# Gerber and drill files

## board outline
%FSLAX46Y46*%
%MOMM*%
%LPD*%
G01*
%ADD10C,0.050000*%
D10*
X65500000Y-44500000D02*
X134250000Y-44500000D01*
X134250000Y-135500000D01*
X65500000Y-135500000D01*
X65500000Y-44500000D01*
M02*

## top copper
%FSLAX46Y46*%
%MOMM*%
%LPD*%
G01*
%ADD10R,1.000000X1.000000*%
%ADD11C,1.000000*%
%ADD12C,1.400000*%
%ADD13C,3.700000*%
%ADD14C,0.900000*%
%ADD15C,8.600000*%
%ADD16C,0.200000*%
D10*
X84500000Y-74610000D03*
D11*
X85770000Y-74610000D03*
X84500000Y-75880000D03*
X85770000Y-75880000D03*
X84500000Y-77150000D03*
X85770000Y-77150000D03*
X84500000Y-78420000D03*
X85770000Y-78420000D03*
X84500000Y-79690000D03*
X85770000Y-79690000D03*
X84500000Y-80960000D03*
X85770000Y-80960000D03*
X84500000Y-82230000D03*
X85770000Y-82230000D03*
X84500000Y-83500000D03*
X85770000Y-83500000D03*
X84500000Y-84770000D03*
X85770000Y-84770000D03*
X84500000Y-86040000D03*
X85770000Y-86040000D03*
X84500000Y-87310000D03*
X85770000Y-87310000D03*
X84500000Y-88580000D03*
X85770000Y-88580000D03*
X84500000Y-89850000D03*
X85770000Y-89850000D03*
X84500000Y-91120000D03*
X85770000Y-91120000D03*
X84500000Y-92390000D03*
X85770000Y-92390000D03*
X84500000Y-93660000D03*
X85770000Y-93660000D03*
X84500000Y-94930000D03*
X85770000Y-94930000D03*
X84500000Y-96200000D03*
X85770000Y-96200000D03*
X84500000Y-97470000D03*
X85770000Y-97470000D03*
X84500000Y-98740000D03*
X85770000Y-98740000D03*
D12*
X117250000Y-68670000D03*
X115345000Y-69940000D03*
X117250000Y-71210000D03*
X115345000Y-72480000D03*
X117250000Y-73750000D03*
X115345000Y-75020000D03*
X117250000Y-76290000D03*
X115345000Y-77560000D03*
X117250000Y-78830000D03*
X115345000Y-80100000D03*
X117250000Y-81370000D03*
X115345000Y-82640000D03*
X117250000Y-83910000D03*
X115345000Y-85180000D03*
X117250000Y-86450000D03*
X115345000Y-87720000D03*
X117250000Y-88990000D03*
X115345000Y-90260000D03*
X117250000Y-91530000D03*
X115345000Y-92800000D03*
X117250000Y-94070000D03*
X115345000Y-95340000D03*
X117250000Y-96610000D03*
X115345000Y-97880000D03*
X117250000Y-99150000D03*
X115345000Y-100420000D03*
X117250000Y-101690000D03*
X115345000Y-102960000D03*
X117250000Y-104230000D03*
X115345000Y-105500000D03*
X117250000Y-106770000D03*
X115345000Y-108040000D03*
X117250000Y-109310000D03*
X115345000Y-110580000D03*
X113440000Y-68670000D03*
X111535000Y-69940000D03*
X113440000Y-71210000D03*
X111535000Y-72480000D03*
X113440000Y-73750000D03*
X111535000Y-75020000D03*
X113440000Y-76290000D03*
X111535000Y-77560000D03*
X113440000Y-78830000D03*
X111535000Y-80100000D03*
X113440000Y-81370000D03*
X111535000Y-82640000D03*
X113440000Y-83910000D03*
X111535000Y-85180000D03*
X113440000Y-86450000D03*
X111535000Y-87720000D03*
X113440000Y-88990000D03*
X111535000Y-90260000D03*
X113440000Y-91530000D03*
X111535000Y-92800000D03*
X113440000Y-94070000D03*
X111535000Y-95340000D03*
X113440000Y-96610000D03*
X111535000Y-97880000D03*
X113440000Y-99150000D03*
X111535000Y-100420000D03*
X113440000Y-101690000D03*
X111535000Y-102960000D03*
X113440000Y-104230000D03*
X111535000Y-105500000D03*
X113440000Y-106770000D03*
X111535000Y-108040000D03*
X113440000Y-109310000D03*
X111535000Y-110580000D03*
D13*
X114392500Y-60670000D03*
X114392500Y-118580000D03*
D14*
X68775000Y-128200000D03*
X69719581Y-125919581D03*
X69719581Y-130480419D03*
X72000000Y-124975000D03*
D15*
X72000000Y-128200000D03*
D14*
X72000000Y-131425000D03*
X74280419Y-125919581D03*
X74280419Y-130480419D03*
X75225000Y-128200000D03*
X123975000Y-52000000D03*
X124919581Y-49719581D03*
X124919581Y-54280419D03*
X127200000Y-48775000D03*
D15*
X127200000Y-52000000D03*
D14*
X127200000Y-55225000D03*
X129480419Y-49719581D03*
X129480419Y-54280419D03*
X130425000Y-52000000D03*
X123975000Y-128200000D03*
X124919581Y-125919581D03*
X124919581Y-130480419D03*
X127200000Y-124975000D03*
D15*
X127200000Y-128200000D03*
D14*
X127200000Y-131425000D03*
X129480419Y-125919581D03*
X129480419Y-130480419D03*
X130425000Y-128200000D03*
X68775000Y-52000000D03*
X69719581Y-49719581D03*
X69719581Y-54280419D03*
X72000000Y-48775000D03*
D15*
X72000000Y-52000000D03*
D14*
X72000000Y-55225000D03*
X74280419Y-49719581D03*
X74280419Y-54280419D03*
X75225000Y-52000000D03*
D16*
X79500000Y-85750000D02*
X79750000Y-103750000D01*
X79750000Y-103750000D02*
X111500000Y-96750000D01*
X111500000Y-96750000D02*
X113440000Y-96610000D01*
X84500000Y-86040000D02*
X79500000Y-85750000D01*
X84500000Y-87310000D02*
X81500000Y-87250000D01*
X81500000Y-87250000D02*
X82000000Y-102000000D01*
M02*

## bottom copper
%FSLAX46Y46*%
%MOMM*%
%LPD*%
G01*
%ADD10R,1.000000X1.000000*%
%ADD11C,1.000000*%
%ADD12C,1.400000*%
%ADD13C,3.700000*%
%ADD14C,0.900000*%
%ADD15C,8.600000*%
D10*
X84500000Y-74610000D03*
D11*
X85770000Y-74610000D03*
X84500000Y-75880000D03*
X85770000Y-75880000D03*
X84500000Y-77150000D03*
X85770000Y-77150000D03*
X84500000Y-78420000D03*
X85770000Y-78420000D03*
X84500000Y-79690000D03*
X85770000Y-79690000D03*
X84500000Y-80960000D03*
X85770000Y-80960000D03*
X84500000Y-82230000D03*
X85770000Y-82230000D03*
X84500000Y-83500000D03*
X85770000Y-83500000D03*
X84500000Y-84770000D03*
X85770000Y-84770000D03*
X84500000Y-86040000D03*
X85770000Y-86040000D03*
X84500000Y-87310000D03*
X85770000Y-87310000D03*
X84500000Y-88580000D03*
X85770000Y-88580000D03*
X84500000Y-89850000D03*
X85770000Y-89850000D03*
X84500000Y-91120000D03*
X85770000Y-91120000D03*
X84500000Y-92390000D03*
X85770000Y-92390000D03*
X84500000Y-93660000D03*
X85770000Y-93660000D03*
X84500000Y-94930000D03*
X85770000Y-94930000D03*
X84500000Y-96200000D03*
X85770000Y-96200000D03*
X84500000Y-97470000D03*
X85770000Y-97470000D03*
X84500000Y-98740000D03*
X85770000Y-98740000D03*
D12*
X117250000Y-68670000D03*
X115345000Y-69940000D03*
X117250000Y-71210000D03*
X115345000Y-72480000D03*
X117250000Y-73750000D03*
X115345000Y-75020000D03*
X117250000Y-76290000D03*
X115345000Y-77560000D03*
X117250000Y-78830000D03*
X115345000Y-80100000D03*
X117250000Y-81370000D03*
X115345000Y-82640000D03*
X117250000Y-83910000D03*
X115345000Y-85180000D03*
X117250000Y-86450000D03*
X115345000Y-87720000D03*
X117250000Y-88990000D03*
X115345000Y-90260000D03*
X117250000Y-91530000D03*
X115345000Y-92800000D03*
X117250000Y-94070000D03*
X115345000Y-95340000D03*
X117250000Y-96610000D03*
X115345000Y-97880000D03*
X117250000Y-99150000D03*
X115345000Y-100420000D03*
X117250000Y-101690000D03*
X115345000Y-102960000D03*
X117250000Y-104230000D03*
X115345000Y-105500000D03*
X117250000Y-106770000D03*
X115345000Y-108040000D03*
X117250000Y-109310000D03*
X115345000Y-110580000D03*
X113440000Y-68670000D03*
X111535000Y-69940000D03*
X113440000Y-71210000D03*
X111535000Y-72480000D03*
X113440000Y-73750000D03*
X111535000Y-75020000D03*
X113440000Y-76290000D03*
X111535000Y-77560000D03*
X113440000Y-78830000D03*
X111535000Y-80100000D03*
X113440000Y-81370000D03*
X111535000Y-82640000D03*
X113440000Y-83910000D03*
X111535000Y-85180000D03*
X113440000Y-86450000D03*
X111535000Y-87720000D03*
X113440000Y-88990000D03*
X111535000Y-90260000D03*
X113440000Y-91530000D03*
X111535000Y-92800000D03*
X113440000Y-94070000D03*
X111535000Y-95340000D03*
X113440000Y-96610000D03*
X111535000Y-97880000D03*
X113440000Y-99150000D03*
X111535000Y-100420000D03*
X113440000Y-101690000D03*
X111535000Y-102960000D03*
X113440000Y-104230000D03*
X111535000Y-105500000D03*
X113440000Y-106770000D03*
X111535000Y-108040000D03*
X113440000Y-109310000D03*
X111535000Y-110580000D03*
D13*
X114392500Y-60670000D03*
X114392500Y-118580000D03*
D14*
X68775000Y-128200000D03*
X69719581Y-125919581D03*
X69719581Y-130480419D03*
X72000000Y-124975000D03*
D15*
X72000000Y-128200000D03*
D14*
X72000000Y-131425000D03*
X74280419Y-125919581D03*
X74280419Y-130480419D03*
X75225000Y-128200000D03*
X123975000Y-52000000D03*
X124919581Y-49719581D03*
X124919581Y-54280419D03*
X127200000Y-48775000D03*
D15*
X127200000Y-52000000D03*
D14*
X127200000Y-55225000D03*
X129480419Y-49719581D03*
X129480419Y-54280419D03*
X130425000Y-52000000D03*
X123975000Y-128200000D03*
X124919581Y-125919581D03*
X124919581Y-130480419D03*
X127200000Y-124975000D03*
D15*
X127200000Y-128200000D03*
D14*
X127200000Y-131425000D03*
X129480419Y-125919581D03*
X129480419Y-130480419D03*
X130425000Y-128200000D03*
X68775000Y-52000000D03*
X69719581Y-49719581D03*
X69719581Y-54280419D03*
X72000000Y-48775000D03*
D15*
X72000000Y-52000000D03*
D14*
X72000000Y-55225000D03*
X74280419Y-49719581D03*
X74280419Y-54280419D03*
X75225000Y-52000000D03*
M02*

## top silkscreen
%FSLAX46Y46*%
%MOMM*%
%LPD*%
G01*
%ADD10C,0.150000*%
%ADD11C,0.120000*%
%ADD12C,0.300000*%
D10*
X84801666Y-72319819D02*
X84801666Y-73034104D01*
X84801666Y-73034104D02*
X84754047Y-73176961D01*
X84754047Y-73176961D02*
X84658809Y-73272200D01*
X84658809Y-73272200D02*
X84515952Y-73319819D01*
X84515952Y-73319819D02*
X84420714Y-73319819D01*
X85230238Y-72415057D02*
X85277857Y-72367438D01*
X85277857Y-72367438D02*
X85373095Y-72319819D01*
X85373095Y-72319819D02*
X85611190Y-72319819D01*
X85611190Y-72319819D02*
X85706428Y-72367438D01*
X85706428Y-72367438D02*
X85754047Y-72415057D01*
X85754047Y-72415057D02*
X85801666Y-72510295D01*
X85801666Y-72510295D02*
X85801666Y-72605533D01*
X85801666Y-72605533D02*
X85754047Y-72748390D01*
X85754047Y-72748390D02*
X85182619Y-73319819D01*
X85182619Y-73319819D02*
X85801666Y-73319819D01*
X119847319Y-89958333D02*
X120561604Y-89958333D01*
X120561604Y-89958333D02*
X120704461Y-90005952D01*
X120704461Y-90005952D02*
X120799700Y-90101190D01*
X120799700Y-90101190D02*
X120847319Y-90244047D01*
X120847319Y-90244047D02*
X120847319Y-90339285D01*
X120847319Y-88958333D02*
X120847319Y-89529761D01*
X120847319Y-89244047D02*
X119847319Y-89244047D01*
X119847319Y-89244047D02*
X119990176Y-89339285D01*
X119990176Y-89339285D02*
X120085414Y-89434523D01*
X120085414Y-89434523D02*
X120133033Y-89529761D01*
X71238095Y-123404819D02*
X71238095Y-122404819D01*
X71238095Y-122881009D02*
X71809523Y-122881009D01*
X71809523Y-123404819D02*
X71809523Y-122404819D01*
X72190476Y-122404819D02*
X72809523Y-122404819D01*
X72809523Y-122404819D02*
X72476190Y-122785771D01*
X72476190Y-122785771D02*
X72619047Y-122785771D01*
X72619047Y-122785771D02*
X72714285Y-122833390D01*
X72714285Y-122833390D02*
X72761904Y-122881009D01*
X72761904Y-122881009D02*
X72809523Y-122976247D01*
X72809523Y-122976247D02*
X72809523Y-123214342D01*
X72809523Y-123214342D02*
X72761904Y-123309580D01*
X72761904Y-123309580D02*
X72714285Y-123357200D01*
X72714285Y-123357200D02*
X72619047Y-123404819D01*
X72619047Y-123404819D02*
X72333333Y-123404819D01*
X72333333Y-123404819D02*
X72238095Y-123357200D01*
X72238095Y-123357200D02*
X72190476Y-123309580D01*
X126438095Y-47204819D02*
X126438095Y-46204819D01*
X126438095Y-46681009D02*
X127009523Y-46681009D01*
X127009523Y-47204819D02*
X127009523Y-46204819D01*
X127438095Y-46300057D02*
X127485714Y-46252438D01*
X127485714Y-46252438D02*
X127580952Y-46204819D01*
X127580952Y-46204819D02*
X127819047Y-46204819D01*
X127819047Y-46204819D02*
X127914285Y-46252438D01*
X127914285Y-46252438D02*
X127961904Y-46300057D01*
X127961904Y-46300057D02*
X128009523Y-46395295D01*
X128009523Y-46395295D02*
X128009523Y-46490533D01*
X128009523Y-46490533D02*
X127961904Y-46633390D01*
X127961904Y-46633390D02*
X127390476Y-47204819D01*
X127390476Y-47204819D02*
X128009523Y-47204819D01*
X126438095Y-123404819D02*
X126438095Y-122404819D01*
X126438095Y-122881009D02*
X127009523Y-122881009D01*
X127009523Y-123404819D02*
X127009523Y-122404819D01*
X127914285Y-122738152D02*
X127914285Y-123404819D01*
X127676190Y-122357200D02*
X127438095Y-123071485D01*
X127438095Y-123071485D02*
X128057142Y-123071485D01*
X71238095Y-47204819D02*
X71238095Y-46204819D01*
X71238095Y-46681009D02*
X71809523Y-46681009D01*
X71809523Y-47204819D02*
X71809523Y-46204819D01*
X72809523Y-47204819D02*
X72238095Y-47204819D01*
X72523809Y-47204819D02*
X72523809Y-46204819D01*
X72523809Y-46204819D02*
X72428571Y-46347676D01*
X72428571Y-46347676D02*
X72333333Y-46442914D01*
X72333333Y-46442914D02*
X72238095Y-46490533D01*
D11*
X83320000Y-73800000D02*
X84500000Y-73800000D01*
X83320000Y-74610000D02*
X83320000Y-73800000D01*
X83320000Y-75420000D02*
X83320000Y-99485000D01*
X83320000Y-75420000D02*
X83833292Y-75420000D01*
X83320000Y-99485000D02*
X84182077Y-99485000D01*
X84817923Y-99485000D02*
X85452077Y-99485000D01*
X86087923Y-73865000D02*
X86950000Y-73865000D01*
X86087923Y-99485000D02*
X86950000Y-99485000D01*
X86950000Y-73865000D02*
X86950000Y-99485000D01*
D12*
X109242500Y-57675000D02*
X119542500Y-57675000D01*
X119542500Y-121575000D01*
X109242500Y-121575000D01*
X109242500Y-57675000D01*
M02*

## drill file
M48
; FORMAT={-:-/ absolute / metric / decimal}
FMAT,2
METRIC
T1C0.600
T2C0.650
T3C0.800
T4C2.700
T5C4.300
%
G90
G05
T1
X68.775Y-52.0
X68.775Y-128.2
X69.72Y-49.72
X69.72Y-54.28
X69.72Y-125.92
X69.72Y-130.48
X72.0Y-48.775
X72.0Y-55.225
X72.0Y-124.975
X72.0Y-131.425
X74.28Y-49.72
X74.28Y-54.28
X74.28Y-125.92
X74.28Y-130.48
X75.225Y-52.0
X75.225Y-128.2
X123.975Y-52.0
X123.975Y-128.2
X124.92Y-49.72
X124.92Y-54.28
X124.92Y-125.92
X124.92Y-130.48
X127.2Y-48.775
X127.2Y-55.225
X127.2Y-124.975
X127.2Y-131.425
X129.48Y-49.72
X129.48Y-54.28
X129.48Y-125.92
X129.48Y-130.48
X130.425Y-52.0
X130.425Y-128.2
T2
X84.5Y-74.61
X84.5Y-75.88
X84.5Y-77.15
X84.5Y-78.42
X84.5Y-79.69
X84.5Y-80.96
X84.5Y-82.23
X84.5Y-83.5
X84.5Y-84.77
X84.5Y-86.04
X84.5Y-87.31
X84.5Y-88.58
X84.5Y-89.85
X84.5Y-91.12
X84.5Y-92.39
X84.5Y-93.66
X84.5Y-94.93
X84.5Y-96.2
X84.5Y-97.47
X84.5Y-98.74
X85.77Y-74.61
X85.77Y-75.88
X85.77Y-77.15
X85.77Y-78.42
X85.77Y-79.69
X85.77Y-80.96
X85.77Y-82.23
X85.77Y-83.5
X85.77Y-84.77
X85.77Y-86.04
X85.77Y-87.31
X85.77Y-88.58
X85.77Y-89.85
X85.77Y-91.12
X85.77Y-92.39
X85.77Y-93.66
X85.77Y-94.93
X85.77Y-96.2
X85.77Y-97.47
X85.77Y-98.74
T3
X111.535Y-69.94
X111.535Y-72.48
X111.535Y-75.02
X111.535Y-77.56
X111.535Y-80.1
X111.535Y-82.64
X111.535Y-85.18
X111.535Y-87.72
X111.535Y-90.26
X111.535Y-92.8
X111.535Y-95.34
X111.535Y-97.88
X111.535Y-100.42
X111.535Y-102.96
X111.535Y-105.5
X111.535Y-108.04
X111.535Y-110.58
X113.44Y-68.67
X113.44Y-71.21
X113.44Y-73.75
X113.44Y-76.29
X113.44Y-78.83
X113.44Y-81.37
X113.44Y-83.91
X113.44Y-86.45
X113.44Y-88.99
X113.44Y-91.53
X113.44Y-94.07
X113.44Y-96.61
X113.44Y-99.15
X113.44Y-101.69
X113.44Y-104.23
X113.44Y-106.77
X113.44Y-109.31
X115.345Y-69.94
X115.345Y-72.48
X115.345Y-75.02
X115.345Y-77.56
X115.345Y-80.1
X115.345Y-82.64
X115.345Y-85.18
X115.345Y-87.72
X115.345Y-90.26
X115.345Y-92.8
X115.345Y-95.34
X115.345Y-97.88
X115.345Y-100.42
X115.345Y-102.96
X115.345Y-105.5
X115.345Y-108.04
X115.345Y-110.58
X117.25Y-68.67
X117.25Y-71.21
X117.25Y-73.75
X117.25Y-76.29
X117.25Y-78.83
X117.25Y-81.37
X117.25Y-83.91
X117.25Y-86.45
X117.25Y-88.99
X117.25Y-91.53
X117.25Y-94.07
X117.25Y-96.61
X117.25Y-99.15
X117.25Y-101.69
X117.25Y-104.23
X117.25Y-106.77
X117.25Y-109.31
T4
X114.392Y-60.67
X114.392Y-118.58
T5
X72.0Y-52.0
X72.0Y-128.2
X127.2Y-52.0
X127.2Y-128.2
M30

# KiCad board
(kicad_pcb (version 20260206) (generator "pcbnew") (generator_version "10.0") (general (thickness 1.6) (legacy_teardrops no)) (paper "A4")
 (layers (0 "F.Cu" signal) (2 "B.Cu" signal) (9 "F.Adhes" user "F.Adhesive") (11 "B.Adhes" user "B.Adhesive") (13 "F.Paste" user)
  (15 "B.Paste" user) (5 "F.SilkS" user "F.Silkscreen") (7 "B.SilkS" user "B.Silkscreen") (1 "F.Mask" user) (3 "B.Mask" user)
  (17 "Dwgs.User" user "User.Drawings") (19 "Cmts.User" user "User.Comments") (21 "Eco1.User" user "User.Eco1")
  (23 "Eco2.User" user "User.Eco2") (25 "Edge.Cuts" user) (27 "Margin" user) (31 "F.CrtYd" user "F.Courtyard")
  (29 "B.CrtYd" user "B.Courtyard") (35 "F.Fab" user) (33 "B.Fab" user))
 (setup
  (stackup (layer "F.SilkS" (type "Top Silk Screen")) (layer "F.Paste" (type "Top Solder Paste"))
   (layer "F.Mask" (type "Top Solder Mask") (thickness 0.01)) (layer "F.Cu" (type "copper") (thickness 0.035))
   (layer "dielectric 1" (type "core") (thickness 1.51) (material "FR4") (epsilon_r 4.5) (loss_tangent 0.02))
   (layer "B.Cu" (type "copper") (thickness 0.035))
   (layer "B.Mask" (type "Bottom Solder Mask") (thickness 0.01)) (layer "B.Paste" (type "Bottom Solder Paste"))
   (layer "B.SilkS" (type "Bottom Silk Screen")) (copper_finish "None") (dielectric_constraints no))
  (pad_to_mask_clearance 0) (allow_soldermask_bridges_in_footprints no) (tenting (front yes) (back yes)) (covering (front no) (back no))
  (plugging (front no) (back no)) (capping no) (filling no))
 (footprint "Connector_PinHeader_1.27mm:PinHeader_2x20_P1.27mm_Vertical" (layer "F.Cu") (at 84.5 74.61)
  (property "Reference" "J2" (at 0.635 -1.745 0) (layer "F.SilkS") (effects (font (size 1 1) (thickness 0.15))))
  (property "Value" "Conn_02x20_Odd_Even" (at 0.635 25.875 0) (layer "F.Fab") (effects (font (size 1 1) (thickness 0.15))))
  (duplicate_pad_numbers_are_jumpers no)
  (fp_line (start -1.18 -0.81) (end 0 -0.81) (stroke (width 0.12) (type solid)) (layer "F.SilkS"))
  (fp_line (start -1.18 0) (end -1.18 -0.81) (stroke (width 0.12) (type solid)) (layer "F.SilkS"))
  (fp_line (start -1.18 0.81) (end -1.18 24.875) (stroke (width 0.12) (type solid)) (layer "F.SilkS"))
  (fp_line (start -1.18 0.81) (end -0.666708 0.81) (stroke (width 0.12) (type solid)) (layer "F.SilkS"))
  (fp_line (start -1.18 24.875) (end -0.317923 24.875) (stroke (width 0.12) (type solid)) (layer "F.SilkS"))
  (fp_line (start 0.317923 24.875) (end 0.952077 24.875) (stroke (width 0.12) (type solid)) (layer "F.SilkS"))
  (fp_line (start 1.587923 -0.745) (end 2.45 -0.745) (stroke (width 0.12) (type solid)) (layer "F.SilkS"))
  (fp_line (start 1.587923 24.875) (end 2.45 24.875) (stroke (width 0.12) (type solid)) (layer "F.SilkS"))
  (fp_line (start 2.45 -0.745) (end 2.45 24.875) (stroke (width 0.12) (type solid)) (layer "F.SilkS"))
  (pad "1" thru_hole rect (at 0 0) (size 1 1) (drill 0.65) (layers "*.Cu" "*.Mask") (remove_unused_layers no) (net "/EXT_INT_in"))
  (pad "2" thru_hole circle (at 1.27 0) (size 1 1) (drill 0.65) (layers "*.Cu" "*.Mask") (remove_unused_layers no) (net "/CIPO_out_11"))
  (pad "3" thru_hole circle (at 0 1.27) (size 1 1) (drill 0.65) (layers "*.Cu" "*.Mask") (remove_unused_layers no) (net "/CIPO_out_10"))
  (pad "4" thru_hole circle (at 1.27 1.27) (size 1 1) (drill 0.65) (layers "*.Cu" "*.Mask") (remove_unused_layers no) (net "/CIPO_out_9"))
  (pad "5" thru_hole circle (at 0 2.54) (size 1 1) (drill 0.65) (layers "*.Cu" "*.Mask") (remove_unused_layers no) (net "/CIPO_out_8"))
  (pad "6" thru_hole circle (at 1.27 2.54) (size 1 1) (drill 0.65) (layers "*.Cu" "*.Mask") (remove_unused_layers no) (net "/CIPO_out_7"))
  (pad "7" thru_hole circle (at 0 3.81) (size 1 1) (drill 0.65) (layers "*.Cu" "*.Mask") (remove_unused_layers no) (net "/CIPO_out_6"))
  (pad "8" thru_hole circle (at 1.27 3.81) (size 1 1) (drill 0.65) (layers "*.Cu" "*.Mask") (remove_unused_layers no) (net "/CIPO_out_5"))
  (pad "9" thru_hole circle (at 0 5.08) (size 1 1) (drill 0.65) (layers "*.Cu" "*.Mask") (remove_unused_layers no) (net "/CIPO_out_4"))
  (pad "10" thru_hole circle (at 1.27 5.08) (size 1 1) (drill 0.65) (layers "*.Cu" "*.Mask") (remove_unused_layers no) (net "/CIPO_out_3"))
  (pad "11" thru_hole circle (at 0 6.35) (size 1 1) (drill 0.65) (layers "*.Cu" "*.Mask") (remove_unused_layers no) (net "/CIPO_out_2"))
  (pad "12" thru_hole circle (at 1.27 6.35) (size 1 1) (drill 0.65) (layers "*.Cu" "*.Mask") (remove_unused_layers no) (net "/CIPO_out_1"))
  (pad "13" thru_hole circle (at 0 7.62) (size 1 1) (drill 0.65) (layers "*.Cu" "*.Mask") (remove_unused_layers no) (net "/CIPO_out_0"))
  (pad "14" thru_hole circle (at 1.27 7.62) (size 1 1) (drill 0.65) (layers "*.Cu" "*.Mask") (remove_unused_layers no) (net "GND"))
  (pad "15" thru_hole circle (at 0 8.89) (size 1 1) (drill 0.65) (layers "*.Cu" "*.Mask") (remove_unused_layers no) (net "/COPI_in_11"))
  (pad "16" thru_hole circle (at 1.27 8.89) (size 1 1) (drill 0.65) (layers "*.Cu" "*.Mask") (remove_unused_layers no) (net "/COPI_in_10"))
  (pad "17" thru_hole circle (at 0 10.16) (size 1 1) (drill 0.65) (layers "*.Cu" "*.Mask") (remove_unused_layers no) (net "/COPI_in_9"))
  (pad "18" thru_hole circle (at 1.27 10.16) (size 1 1) (drill 0.65) (layers "*.Cu" "*.Mask") (remove_unused_layers no) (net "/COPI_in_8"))
  (pad "19" thru_hole circle (at 0 11.43) (size 1 1) (drill 0.65) (layers "*.Cu" "*.Mask") (remove_unused_layers no) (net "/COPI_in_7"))
  (pad "20" thru_hole circle (at 1.27 11.43) (size 1 1) (drill 0.65) (layers "*.Cu" "*.Mask") (remove_unused_layers no) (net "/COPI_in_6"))
  (pad "21" thru_hole circle (at 0 12.7) (size 1 1) (drill 0.65) (layers "*.Cu" "*.Mask") (remove_unused_layers no) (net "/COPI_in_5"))
  (pad "22" thru_hole circle (at 1.27 12.7) (size 1 1) (drill 0.65) (layers "*.Cu" "*.Mask") (remove_unused_layers no) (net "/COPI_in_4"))
  (pad "23" thru_hole circle (at 0 13.97) (size 1 1) (drill 0.65) (layers "*.Cu" "*.Mask") (remove_unused_layers no) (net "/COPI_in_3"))
  (pad "24" thru_hole circle (at 1.27 13.97) (size 1 1) (drill 0.65) (layers "*.Cu" "*.Mask") (remove_unused_layers no) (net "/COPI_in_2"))
  (pad "25" thru_hole circle (at 0 15.24) (size 1 1) (drill 0.65) (layers "*.Cu" "*.Mask") (remove_unused_layers no) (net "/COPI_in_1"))
  (pad "26" thru_hole circle (at 1.27 15.24) (size 1 1) (drill 0.65) (layers "*.Cu" "*.Mask") (remove_unused_layers no) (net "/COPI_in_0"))
  (pad "27" thru_hole circle (at 0 16.51) (size 1 1) (drill 0.65) (layers "*.Cu" "*.Mask") (remove_unused_layers no) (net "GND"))
  (pad "28" thru_hole circle (at 1.27 16.51) (size 1 1) (drill 0.65) (layers "*.Cu" "*.Mask") (remove_unused_layers no) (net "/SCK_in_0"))
  (pad "29" thru_hole circle (at 0 17.78) (size 1 1) (drill 0.65) (layers "*.Cu" "*.Mask") (remove_unused_layers no) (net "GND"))
  (pad "30" thru_hole circle (at 1.27 17.78) (size 1 1) (drill 0.65) (layers "*.Cu" "*.Mask") (remove_unused_layers no) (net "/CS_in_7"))
  (pad "31" thru_hole circle (at 0 19.05) (size 1 1) (drill 0.65) (layers "*.Cu" "*.Mask") (remove_unused_layers no) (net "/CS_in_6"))
  (pad "32" thru_hole circle (at 1.27 19.05) (size 1 1) (drill 0.65) (layers "*.Cu" "*.Mask") (remove_unused_layers no) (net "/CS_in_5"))
  (pad "33" thru_hole circle (at 0 20.32) (size 1 1) (drill 0.65) (layers "*.Cu" "*.Mask") (remove_unused_layers no) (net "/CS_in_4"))
  (pad "34" thru_hole circle (at 1.27 20.32) (size 1 1) (drill 0.65) (layers "*.Cu" "*.Mask") (remove_unused_layers no) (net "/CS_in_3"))
  (pad "35" thru_hole circle (at 0 21.59) (size 1 1) (drill 0.65) (layers "*.Cu" "*.Mask") (remove_unused_layers no) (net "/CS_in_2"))
  (pad "36" thru_hole circle (at 1.27 21.59) (size 1 1) (drill 0.65) (layers "*.Cu" "*.Mask") (remove_unused_layers no) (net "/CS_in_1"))
  (pad "37" thru_hole circle (at 0 22.86) (size 1 1) (drill 0.65) (layers "*.Cu" "*.Mask") (remove_unused_layers no) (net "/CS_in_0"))
  (pad "38" thru_hole circle (at 1.27 22.86) (size 1 1) (drill 0.65) (layers "*.Cu" "*.Mask") (remove_unused_layers no) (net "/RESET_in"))
  (pad "39" thru_hole circle (at 0 24.13) (size 1 1) (drill 0.65) (layers "*.Cu" "*.Mask") (remove_unused_layers no) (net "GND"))
  (pad "40" thru_hole circle (at 1.27 24.13) (size 1 1) (drill 0.65) (layers "*.Cu" "*.Mask") (remove_unused_layers no) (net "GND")))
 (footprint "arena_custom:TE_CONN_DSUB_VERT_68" (layer "F.Cu") (at 114.3925 89.625 -90)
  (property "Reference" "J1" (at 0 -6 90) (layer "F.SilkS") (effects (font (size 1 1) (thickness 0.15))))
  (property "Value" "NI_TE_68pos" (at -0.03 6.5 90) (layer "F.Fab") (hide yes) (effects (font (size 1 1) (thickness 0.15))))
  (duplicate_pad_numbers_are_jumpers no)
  (fp_rect (start -31.95 -5.15) (end 31.95 5.15) (stroke (width 0.3) (type default)) (fill no) (layer "F.SilkS"))
  (pad "1" thru_hole circle (at -20.955 -2.8575 270) (size 1.4 1.4) (drill 0.8) (layers "*.Cu" "*.Mask") (remove_unused_layers no)
   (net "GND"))
  (pad "2" thru_hole circle (at -19.685 -0.9525 270) (size 1.4 1.4) (drill 0.8) (layers "*.Cu" "*.Mask") (remove_unused_layers no)
   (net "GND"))
  (pad "3" thru_hole circle (at -18.415 -2.8575 270) (size 1.4 1.4) (drill 0.8) (layers "*.Cu" "*.Mask") (remove_unused_layers no)
   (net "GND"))
  (pad "4" thru_hole circle (at -17.145 -0.9525 270) (size 1.4 1.4) (drill 0.8) (layers "*.Cu" "*.Mask") (remove_unused_layers no)
   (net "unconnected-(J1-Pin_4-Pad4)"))
  (pad "5" thru_hole circle (at -15.875 -2.8575 270) (size 1.4 1.4) (drill 0.8) (layers "*.Cu" "*.Mask") (remove_unused_layers no)
   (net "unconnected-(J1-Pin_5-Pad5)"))
  (pad "6" thru_hole circle (at -14.605 -0.9525 270) (size 1.4 1.4) (drill 0.8) (layers "*.Cu" "*.Mask") (remove_unused_layers no)
   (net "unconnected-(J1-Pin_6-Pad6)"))
  (pad "7" thru_hole circle (at -13.335 -2.8575 270) (size 1.4 1.4) (drill 0.8) (layers "*.Cu" "*.Mask") (remove_unused_layers no)
   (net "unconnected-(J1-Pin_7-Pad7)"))
  (pad "8" thru_hole circle (at -12.065 -0.9525 270) (size 1.4 1.4) (drill 0.8) (layers "*.Cu" "*.Mask") (remove_unused_layers no)
   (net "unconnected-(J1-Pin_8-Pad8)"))
  (pad "9" thru_hole circle (at -10.795 -2.8575 270) (size 1.4 1.4) (drill 0.8) (layers "*.Cu" "*.Mask") (remove_unused_layers no)
   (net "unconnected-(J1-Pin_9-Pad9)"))
  (pad "10" thru_hole circle (at -9.525 -0.9525 270) (size 1.4 1.4) (drill 0.8) (layers "*.Cu" "*.Mask") (remove_unused_layers no)
   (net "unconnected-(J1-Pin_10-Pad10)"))
  (pad "11" thru_hole circle (at -8.255 -2.8575 270) (size 1.4 1.4) (drill 0.8) (layers "*.Cu" "*.Mask") (remove_unused_layers no)
   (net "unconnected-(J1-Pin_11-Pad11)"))
  (pad "12" thru_hole circle (at -6.985 -0.9525 270) (size 1.4 1.4) (drill 0.8) (layers "*.Cu" "*.Mask") (remove_unused_layers no)
   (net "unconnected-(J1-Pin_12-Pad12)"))
  (pad "13" thru_hole circle (at -5.715 -2.8575 270) (size 1.4 1.4) (drill 0.8) (layers "*.Cu" "*.Mask") (remove_unused_layers no)
   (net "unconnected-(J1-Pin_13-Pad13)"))
  (pad "14" thru_hole circle (at -4.445 -0.9525 270) (size 1.4 1.4) (drill 0.8) (layers "*.Cu" "*.Mask") (remove_unused_layers no)
   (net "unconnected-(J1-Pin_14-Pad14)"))
  (pad "15" thru_hole circle (at -3.175 -2.8575 270) (size 1.4 1.4) (drill 0.8) (layers "*.Cu" "*.Mask") (remove_unused_layers no)
   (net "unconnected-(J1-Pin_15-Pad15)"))
  (pad "16" thru_hole circle (at -1.905 -0.9525 270) (size 1.4 1.4) (drill 0.8) (layers "*.Cu" "*.Mask") (remove_unused_layers no)
   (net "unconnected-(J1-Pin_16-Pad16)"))
  (pad "17" thru_hole circle (at -0.635 -2.8575 270) (size 1.4 1.4) (drill 0.8) (layers "*.Cu" "*.Mask") (remove_unused_layers no)
   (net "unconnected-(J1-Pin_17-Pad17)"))
  (pad "18" thru_hole circle (at 0.635 -0.9525 270) (size 1.4 1.4) (drill 0.8) (layers "*.Cu" "*.Mask") (remove_unused_layers no)
   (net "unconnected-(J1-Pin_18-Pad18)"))
  (pad "19" thru_hole circle (at 1.905 -2.8575 270) (size 1.4 1.4) (drill 0.8) (layers "*.Cu" "*.Mask") (remove_unused_layers no)
   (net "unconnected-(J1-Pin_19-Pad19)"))
  (pad "20" thru_hole circle (at 3.175 -0.9525 270) (size 1.4 1.4) (drill 0.8) (layers "*.Cu" "*.Mask") (remove_unused_layers no)
   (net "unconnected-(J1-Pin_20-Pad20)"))
  (pad "21" thru_hole circle (at 4.445 -2.8575 270) (size 1.4 1.4) (drill 0.8) (layers "*.Cu" "*.Mask") (remove_unused_layers no)
   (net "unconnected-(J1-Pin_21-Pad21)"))
  (pad "22" thru_hole circle (at 5.715 -0.9525 270) (size 1.4 1.4) (drill 0.8) (layers "*.Cu" "*.Mask") (remove_unused_layers no)
   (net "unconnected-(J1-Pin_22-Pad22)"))
  (pad "23" thru_hole circle (at 6.985 -2.8575 270) (size 1.4 1.4) (drill 0.8) (layers "*.Cu" "*.Mask") (remove_unused_layers no)
   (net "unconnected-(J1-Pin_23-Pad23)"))
  (pad "24" thru_hole circle (at 8.255 -0.9525 270) (size 1.4 1.4) (drill 0.8) (layers "*.Cu" "*.Mask") (remove_unused_layers no)
   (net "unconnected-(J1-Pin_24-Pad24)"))
  (pad "25" thru_hole circle (at 9.525 -2.8575 270) (size 1.4 1.4) (drill 0.8) (layers "*.Cu" "*.Mask") (remove_unused_layers no)
   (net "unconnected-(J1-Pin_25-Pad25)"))
  (pad "26" thru_hole circle (at 10.795 -0.9525 270) (size 1.4 1.4) (drill 0.8) (layers "*.Cu" "*.Mask") (remove_unused_layers no)
   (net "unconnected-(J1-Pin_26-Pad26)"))
  (pad "27" thru_hole circle (at 12.065 -2.8575 270) (size 1.4 1.4) (drill 0.8) (layers "*.Cu" "*.Mask") (remove_unused_layers no)
   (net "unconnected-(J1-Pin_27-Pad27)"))
  (pad "28" thru_hole circle (at 13.335 -0.9525 270) (size 1.4 1.4) (drill 0.8) (layers "*.Cu" "*.Mask") (remove_unused_layers no)
   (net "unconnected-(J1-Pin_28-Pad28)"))
  (pad "29" thru_hole circle (at 14.605 -2.8575 270) (size 1.4 1.4) (drill 0.8) (layers "*.Cu" "*.Mask") (remove_unused_layers no)
   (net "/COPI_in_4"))
  (pad "30" thru_hole circle (at 15.875 -0.9525 270) (size 1.4 1.4) (drill 0.8) (layers "*.Cu" "*.Mask") (remove_unused_layers no)
   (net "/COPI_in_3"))
  (pad "31" thru_hole circle (at 17.145 -2.8575 270) (size 1.4 1.4) (drill 0.8) (layers "*.Cu" "*.Mask") (remove_unused_layers no)
   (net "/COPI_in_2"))
  (pad "32" thru_hole circle (at 18.415 -0.9525 270) (size 1.4 1.4) (drill 0.8) (layers "*.Cu" "*.Mask") (remove_unused_layers no)
   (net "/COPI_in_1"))
  (pad "33" thru_hole circle (at 19.685 -2.8575 270) (size 1.4 1.4) (drill 0.8) (layers "*.Cu" "*.Mask") (remove_unused_layers no)
   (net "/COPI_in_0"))
  (pad "34" thru_hole circle (at 20.955 -0.9525 270) (size 1.4 1.4) (drill 0.8) (layers "*.Cu" "*.Mask") (remove_unused_layers no)
   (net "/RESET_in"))
  (pad "35" thru_hole circle (at -20.955 0.9525 270) (size 1.4 1.4) (drill 0.8) (layers "*.Cu" "*.Mask") (remove_unused_layers no)
   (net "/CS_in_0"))
  (pad "36" thru_hole circle (at -19.685 2.8575 270) (size 1.4 1.4) (drill 0.8) (layers "*.Cu" "*.Mask") (remove_unused_layers no)
   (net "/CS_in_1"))
  (pad "37" thru_hole circle (at -18.415 0.9525 270) (size 1.4 1.4) (drill 0.8) (layers "*.Cu" "*.Mask") (remove_unused_layers no)
   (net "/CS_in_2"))
  (pad "38" thru_hole circle (at -17.145 2.8575 270) (size 1.4 1.4) (drill 0.8) (layers "*.Cu" "*.Mask") (remove_unused_layers no)
   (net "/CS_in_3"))
  (pad "39" thru_hole circle (at -15.875 0.9525 270) (size 1.4 1.4) (drill 0.8) (layers "*.Cu" "*.Mask") (remove_unused_layers no)
   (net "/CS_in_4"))
  (pad "40" thru_hole circle (at -14.605 2.8575 270) (size 1.4 1.4) (drill 0.8) (layers "*.Cu" "*.Mask") (remove_unused_layers no)
   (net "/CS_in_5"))
  (pad "41" thru_hole circle (at -13.335 0.9525 270) (size 1.4 1.4) (drill 0.8) (layers "*.Cu" "*.Mask") (remove_unused_layers no)
   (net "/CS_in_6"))
  (pad "42" thru_hole circle (at -12.065 2.8575 270) (size 1.4 1.4) (drill 0.8) (layers "*.Cu" "*.Mask") (remove_unused_layers no)
   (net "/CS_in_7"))
  (pad "43" thru_hole circle (at -10.795 0.9525 270) (size 1.4 1.4) (drill 0.8) (layers "*.Cu" "*.Mask") (remove_unused_layers no)
   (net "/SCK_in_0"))
  (pad "44" thru_hole circle (at -9.525 2.8575 270) (size 1.4 1.4) (drill 0.8) (layers "*.Cu" "*.Mask") (remove_unused_layers no)
   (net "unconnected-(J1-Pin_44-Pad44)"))
  (pad "45" thru_hole circle (at -8.255 0.9525 270) (size 1.4 1.4) (drill 0.8) (layers "*.Cu" "*.Mask") (remove_unused_layers no)
   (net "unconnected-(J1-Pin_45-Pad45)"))
  (pad "46" thru_hole circle (at -6.985 2.8575 270) (size 1.4 1.4) (drill 0.8) (layers "*.Cu" "*.Mask") (remove_unused_layers no)
   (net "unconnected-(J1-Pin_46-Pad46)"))
  (pad "47" thru_hole circle (at -5.715 0.9525 270) (size 1.4 1.4) (drill 0.8) (layers "*.Cu" "*.Mask") (remove_unused_layers no)
   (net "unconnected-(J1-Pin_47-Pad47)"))
  (pad "48" thru_hole circle (at -4.445 2.8575 270) (size 1.4 1.4) (drill 0.8) (layers "*.Cu" "*.Mask") (remove_unused_layers no)
   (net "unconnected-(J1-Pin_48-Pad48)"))
  (pad "49" thru_hole circle (at -3.175 0.9525 270) (size 1.4 1.4) (drill 0.8) (layers "*.Cu" "*.Mask") (remove_unused_layers no)
   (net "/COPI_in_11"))
  (pad "50" thru_hole circle (at -1.905 2.8575 270) (size 1.4 1.4) (drill 0.8) (layers "*.Cu" "*.Mask") (remove_unused_layers no)
   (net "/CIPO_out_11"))
  (pad "51" thru_hole circle (at -0.635 0.9525 270) (size 1.4 1.4) (drill 0.8) (layers "*.Cu" "*.Mask") (remove_unused_layers no)
   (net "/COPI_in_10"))
  (pad "52" thru_hole circle (at 0.635 2.8575 270) (size 1.4 1.4) (drill 0.8) (layers "*.Cu" "*.Mask") (remove_unused_layers no)
   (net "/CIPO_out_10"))
  (pad "53" thru_hole circle (at 1.905 0.9525 270) (size 1.4 1.4) (drill 0.8) (layers "*.Cu" "*.Mask") (remove_unused_layers no)
   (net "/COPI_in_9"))
  (pad "54" thru_hole circle (at 3.175 2.8575 270) (size 1.4 1.4) (drill 0.8) (layers "*.Cu" "*.Mask") (remove_unused_layers no)
   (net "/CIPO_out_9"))
  (pad "55" thru_hole circle (at 4.445 0.9525 270) (size 1.4 1.4) (drill 0.8) (layers "*.Cu" "*.Mask") (remove_unused_layers no)
   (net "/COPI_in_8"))
  (pad "56" thru_hole circle (at 5.715 2.8575 270) (size 1.4 1.4) (drill 0.8) (layers "*.Cu" "*.Mask") (remove_unused_layers no)
   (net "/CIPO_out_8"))
  (pad "57" thru_hole circle (at 6.985 0.9525 270) (size 1.4 1.4) (drill 0.8) (layers "*.Cu" "*.Mask") (remove_unused_layers no)
   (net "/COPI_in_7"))
  (pad "58" thru_hole circle (at 8.255 2.8575 270) (size 1.4 1.4) (drill 0.8) (layers "*.Cu" "*.Mask") (remove_unused_layers no)
   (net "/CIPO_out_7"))
  (pad "59" thru_hole circle (at 9.525 0.9525 270) (size 1.4 1.4) (drill 0.8) (layers "*.Cu" "*.Mask") (remove_unused_layers no)
   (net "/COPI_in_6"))
  (pad "60" thru_hole circle (at 10.795 2.8575 270) (size 1.4 1.4) (drill 0.8) (layers "*.Cu" "*.Mask") (remove_unused_layers no)
   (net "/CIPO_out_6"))
  (pad "61" thru_hole circle (at 12.065 0.9525 270) (size 1.4 1.4) (drill 0.8) (layers "*.Cu" "*.Mask") (remove_unused_layers no)
   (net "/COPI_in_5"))
  (pad "62" thru_hole circle (at 13.335 2.8575 270) (size 1.4 1.4) (drill 0.8) (layers "*.Cu" "*.Mask") (remove_unused_layers no)
   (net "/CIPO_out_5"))
  (pad "63" thru_hole circle (at 14.605 0.9525 270) (size 1.4 1.4) (drill 0.8) (layers "*.Cu" "*.Mask") (remove_unused_layers no)
   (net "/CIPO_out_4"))
  (pad "64" thru_hole circle (at 15.875 2.8575 270) (size 1.4 1.4) (drill 0.8) (layers "*.Cu" "*.Mask") (remove_unused_layers no)
   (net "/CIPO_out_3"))
  (pad "65" thru_hole circle (at 17.145 0.9525 270) (size 1.4 1.4) (drill 0.8) (layers "*.Cu" "*.Mask") (remove_unused_layers no)
   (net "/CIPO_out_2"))
  (pad "66" thru_hole circle (at 18.415 2.8575 270) (size 1.4 1.4) (drill 0.8) (layers "*.Cu" "*.Mask") (remove_unused_layers no)
   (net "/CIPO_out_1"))
  (pad "67" thru_hole circle (at 19.685 0.9525 270) (size 1.4 1.4) (drill 0.8) (layers "*.Cu" "*.Mask") (remove_unused_layers no)
   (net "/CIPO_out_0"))
  (pad "68" thru_hole circle (at 20.955 2.8575 270) (size 1.4 1.4) (drill 0.8) (layers "*.Cu" "*.Mask") (remove_unused_layers no)
   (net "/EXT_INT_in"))
  (pad "69" thru_hole circle (at -28.955 0 270) (size 3.7 3.7) (drill 2.7) (layers "*.Cu" "*.Mask") (remove_unused_layers no) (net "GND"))
  (pad "70" thru_hole circle (at 28.955 0 270) (size 3.7 3.7) (drill 2.7) (layers "*.Cu" "*.Mask") (remove_unused_layers no) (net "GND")))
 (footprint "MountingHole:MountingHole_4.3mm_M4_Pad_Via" (layer "F.Cu") (at 72 128.2)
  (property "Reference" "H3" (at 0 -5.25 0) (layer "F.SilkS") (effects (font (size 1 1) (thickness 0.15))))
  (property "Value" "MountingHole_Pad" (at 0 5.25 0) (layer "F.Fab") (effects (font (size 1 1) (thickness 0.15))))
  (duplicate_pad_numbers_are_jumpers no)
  (pad "1" thru_hole circle (at -3.225 0) (size 0.9 0.9) (drill 0.6) (layers "*.Cu" "*.Mask") (remove_unused_layers no) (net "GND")
   (zone_connect 2))
  (pad "1" thru_hole circle (at -2.280419 -2.280419) (size 0.9 0.9) (drill 0.6) (layers "*.Cu" "*.Mask") (remove_unused_layers no)
   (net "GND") (zone_connect 2))
  (pad "1" thru_hole circle (at -2.280419 2.280419) (size 0.9 0.9) (drill 0.6) (layers "*.Cu" "*.Mask") (remove_unused_layers no)
   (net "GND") (zone_connect 2))
  (pad "1" thru_hole circle (at 0 -3.225) (size 0.9 0.9) (drill 0.6) (layers "*.Cu" "*.Mask") (remove_unused_layers no) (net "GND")
   (zone_connect 2))
  (pad "1" thru_hole circle (at 0 0) (size 8.6 8.6) (drill 4.3) (layers "*.Cu" "*.Mask") (remove_unused_layers no) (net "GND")
   (zone_connect 2))
  (pad "1" thru_hole circle (at 0 3.225) (size 0.9 0.9) (drill 0.6) (layers "*.Cu" "*.Mask") (remove_unused_layers no) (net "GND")
   (zone_connect 2))
  (pad "1" thru_hole circle (at 2.280419 -2.280419) (size 0.9 0.9) (drill 0.6) (layers "*.Cu" "*.Mask") (remove_unused_layers no)
   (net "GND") (zone_connect 2))
  (pad "1" thru_hole circle (at 2.280419 2.280419) (size 0.9 0.9) (drill 0.6) (layers "*.Cu" "*.Mask") (remove_unused_layers no) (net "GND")
   (zone_connect 2))
  (pad "1" thru_hole circle (at 3.225 0) (size 0.9 0.9) (drill 0.6) (layers "*.Cu" "*.Mask") (remove_unused_layers no) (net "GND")
   (zone_connect 2)))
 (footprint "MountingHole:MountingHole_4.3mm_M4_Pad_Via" (layer "F.Cu") (at 127.2 52)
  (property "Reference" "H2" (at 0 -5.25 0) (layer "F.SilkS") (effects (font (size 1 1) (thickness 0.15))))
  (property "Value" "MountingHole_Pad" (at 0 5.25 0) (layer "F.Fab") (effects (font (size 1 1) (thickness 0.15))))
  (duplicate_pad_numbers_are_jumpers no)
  (pad "1" thru_hole circle (at -3.225 0) (size 0.9 0.9) (drill 0.6) (layers "*.Cu" "*.Mask") (remove_unused_layers no) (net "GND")
   (zone_connect 2))
  (pad "1" thru_hole circle (at -2.280419 -2.280419) (size 0.9 0.9) (drill 0.6) (layers "*.Cu" "*.Mask") (remove_unused_layers no)
   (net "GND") (zone_connect 2))
  (pad "1" thru_hole circle (at -2.280419 2.280419) (size 0.9 0.9) (drill 0.6) (layers "*.Cu" "*.Mask") (remove_unused_layers no)
   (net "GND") (zone_connect 2))
  (pad "1" thru_hole circle (at 0 -3.225) (size 0.9 0.9) (drill 0.6) (layers "*.Cu" "*.Mask") (remove_unused_layers no) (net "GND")
   (zone_connect 2))
  (pad "1" thru_hole circle (at 0 0) (size 8.6 8.6) (drill 4.3) (layers "*.Cu" "*.Mask") (remove_unused_layers no) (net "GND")
   (zone_connect 2))
  (pad "1" thru_hole circle (at 0 3.225) (size 0.9 0.9) (drill 0.6) (layers "*.Cu" "*.Mask") (remove_unused_layers no) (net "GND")
   (zone_connect 2))
  (pad "1" thru_hole circle (at 2.280419 -2.280419) (size 0.9 0.9) (drill 0.6) (layers "*.Cu" "*.Mask") (remove_unused_layers no)
   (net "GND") (zone_connect 2))
  (pad "1" thru_hole circle (at 2.280419 2.280419) (size 0.9 0.9) (drill 0.6) (layers "*.Cu" "*.Mask") (remove_unused_layers no) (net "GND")
   (zone_connect 2))
  (pad "1" thru_hole circle (at 3.225 0) (size 0.9 0.9) (drill 0.6) (layers "*.Cu" "*.Mask") (remove_unused_layers no) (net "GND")
   (zone_connect 2)))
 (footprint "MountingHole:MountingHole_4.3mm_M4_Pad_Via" (layer "F.Cu") (at 127.2 128.2)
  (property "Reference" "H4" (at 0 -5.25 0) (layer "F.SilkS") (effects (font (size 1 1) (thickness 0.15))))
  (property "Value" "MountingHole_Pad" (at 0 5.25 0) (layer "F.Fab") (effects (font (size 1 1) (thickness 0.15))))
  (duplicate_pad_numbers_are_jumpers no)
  (pad "1" thru_hole circle (at -3.225 0) (size 0.9 0.9) (drill 0.6) (layers "*.Cu" "*.Mask") (remove_unused_layers no) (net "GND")
   (zone_connect 2))
  (pad "1" thru_hole circle (at -2.280419 -2.280419) (size 0.9 0.9) (drill 0.6) (layers "*.Cu" "*.Mask") (remove_unused_layers no)
   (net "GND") (zone_connect 2))
  (pad "1" thru_hole circle (at -2.280419 2.280419) (size 0.9 0.9) (drill 0.6) (layers "*.Cu" "*.Mask") (remove_unused_layers no)
   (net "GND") (zone_connect 2))
  (pad "1" thru_hole circle (at 0 -3.225) (size 0.9 0.9) (drill 0.6) (layers "*.Cu" "*.Mask") (remove_unused_layers no) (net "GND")
   (zone_connect 2))
  (pad "1" thru_hole circle (at 0 0) (size 8.6 8.6) (drill 4.3) (layers "*.Cu" "*.Mask") (remove_unused_layers no) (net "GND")
   (zone_connect 2))
  (pad "1" thru_hole circle (at 0 3.225) (size 0.9 0.9) (drill 0.6) (layers "*.Cu" "*.Mask") (remove_unused_layers no) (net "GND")
   (zone_connect 2))
  (pad "1" thru_hole circle (at 2.280419 -2.280419) (size 0.9 0.9) (drill 0.6) (layers "*.Cu" "*.Mask") (remove_unused_layers no)
   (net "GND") (zone_connect 2))
  (pad "1" thru_hole circle (at 2.280419 2.280419) (size 0.9 0.9) (drill 0.6) (layers "*.Cu" "*.Mask") (remove_unused_layers no) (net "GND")
   (zone_connect 2))
  (pad "1" thru_hole circle (at 3.225 0) (size 0.9 0.9) (drill 0.6) (layers "*.Cu" "*.Mask") (remove_unused_layers no) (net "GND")
   (zone_connect 2)))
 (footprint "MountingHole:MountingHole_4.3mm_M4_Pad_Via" (layer "F.Cu") (at 72 52)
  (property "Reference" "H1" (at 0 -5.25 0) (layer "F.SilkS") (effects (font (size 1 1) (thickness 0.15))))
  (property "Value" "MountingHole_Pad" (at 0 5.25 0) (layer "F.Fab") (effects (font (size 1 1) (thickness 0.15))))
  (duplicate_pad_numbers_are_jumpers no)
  (pad "1" thru_hole circle (at -3.225 0) (size 0.9 0.9) (drill 0.6) (layers "*.Cu" "*.Mask") (remove_unused_layers no) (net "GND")
   (zone_connect 2))
  (pad "1" thru_hole circle (at -2.280419 -2.280419) (size 0.9 0.9) (drill 0.6) (layers "*.Cu" "*.Mask") (remove_unused_layers no)
   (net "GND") (zone_connect 2))
  (pad "1" thru_hole circle (at -2.280419 2.280419) (size 0.9 0.9) (drill 0.6) (layers "*.Cu" "*.Mask") (remove_unused_layers no)
   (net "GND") (zone_connect 2))
  (pad "1" thru_hole circle (at 0 -3.225) (size 0.9 0.9) (drill 0.6) (layers "*.Cu" "*.Mask") (remove_unused_layers no) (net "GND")
   (zone_connect 2))
  (pad "1" thru_hole circle (at 0 0) (size 8.6 8.6) (drill 4.3) (layers "*.Cu" "*.Mask") (remove_unused_layers no) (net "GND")
   (zone_connect 2))
  (pad "1" thru_hole circle (at 0 3.225) (size 0.9 0.9) (drill 0.6) (layers "*.Cu" "*.Mask") (remove_unused_layers no) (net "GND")
   (zone_connect 2))
  (pad "1" thru_hole circle (at 2.280419 -2.280419) (size 0.9 0.9) (drill 0.6) (layers "*.Cu" "*.Mask") (remove_unused_layers no)
   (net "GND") (zone_connect 2))
  (pad "1" thru_hole circle (at 2.280419 2.280419) (size 0.9 0.9) (drill 0.6) (layers "*.Cu" "*.Mask") (remove_unused_layers no) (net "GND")
   (zone_connect 2))
  (pad "1" thru_hole circle (at 3.225 0) (size 0.9 0.9) (drill 0.6) (layers "*.Cu" "*.Mask") (remove_unused_layers no) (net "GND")
   (zone_connect 2)))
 (gr_rect (start 65.5 44.5) (end 134.25 135.5) (stroke (width 0.05) (type default)) (fill no) (layer "Edge.Cuts"))
 (segment (start 79.5 85.75) (end 79.75 103.75) (width 0.2) (layer "F.Cu") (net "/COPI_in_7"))
 (segment (start 79.75 103.75) (end 111.5 96.75) (width 0.2) (layer "F.Cu") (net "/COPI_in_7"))
 (segment (start 111.5 96.75) (end 113.44 96.61) (width 0.2) (layer "F.Cu") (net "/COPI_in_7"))
 (segment (start 84.5 86.04) (end 79.5 85.75) (width 0.2) (layer "F.Cu") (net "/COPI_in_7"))
 (segment (start 84.5 87.31) (end 81.5 87.25) (width 0.2) (layer "F.Cu") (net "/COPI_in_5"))
 (segment (start 81.5 87.25) (end 82 102) (width 0.2) (layer "F.Cu") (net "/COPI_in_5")))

